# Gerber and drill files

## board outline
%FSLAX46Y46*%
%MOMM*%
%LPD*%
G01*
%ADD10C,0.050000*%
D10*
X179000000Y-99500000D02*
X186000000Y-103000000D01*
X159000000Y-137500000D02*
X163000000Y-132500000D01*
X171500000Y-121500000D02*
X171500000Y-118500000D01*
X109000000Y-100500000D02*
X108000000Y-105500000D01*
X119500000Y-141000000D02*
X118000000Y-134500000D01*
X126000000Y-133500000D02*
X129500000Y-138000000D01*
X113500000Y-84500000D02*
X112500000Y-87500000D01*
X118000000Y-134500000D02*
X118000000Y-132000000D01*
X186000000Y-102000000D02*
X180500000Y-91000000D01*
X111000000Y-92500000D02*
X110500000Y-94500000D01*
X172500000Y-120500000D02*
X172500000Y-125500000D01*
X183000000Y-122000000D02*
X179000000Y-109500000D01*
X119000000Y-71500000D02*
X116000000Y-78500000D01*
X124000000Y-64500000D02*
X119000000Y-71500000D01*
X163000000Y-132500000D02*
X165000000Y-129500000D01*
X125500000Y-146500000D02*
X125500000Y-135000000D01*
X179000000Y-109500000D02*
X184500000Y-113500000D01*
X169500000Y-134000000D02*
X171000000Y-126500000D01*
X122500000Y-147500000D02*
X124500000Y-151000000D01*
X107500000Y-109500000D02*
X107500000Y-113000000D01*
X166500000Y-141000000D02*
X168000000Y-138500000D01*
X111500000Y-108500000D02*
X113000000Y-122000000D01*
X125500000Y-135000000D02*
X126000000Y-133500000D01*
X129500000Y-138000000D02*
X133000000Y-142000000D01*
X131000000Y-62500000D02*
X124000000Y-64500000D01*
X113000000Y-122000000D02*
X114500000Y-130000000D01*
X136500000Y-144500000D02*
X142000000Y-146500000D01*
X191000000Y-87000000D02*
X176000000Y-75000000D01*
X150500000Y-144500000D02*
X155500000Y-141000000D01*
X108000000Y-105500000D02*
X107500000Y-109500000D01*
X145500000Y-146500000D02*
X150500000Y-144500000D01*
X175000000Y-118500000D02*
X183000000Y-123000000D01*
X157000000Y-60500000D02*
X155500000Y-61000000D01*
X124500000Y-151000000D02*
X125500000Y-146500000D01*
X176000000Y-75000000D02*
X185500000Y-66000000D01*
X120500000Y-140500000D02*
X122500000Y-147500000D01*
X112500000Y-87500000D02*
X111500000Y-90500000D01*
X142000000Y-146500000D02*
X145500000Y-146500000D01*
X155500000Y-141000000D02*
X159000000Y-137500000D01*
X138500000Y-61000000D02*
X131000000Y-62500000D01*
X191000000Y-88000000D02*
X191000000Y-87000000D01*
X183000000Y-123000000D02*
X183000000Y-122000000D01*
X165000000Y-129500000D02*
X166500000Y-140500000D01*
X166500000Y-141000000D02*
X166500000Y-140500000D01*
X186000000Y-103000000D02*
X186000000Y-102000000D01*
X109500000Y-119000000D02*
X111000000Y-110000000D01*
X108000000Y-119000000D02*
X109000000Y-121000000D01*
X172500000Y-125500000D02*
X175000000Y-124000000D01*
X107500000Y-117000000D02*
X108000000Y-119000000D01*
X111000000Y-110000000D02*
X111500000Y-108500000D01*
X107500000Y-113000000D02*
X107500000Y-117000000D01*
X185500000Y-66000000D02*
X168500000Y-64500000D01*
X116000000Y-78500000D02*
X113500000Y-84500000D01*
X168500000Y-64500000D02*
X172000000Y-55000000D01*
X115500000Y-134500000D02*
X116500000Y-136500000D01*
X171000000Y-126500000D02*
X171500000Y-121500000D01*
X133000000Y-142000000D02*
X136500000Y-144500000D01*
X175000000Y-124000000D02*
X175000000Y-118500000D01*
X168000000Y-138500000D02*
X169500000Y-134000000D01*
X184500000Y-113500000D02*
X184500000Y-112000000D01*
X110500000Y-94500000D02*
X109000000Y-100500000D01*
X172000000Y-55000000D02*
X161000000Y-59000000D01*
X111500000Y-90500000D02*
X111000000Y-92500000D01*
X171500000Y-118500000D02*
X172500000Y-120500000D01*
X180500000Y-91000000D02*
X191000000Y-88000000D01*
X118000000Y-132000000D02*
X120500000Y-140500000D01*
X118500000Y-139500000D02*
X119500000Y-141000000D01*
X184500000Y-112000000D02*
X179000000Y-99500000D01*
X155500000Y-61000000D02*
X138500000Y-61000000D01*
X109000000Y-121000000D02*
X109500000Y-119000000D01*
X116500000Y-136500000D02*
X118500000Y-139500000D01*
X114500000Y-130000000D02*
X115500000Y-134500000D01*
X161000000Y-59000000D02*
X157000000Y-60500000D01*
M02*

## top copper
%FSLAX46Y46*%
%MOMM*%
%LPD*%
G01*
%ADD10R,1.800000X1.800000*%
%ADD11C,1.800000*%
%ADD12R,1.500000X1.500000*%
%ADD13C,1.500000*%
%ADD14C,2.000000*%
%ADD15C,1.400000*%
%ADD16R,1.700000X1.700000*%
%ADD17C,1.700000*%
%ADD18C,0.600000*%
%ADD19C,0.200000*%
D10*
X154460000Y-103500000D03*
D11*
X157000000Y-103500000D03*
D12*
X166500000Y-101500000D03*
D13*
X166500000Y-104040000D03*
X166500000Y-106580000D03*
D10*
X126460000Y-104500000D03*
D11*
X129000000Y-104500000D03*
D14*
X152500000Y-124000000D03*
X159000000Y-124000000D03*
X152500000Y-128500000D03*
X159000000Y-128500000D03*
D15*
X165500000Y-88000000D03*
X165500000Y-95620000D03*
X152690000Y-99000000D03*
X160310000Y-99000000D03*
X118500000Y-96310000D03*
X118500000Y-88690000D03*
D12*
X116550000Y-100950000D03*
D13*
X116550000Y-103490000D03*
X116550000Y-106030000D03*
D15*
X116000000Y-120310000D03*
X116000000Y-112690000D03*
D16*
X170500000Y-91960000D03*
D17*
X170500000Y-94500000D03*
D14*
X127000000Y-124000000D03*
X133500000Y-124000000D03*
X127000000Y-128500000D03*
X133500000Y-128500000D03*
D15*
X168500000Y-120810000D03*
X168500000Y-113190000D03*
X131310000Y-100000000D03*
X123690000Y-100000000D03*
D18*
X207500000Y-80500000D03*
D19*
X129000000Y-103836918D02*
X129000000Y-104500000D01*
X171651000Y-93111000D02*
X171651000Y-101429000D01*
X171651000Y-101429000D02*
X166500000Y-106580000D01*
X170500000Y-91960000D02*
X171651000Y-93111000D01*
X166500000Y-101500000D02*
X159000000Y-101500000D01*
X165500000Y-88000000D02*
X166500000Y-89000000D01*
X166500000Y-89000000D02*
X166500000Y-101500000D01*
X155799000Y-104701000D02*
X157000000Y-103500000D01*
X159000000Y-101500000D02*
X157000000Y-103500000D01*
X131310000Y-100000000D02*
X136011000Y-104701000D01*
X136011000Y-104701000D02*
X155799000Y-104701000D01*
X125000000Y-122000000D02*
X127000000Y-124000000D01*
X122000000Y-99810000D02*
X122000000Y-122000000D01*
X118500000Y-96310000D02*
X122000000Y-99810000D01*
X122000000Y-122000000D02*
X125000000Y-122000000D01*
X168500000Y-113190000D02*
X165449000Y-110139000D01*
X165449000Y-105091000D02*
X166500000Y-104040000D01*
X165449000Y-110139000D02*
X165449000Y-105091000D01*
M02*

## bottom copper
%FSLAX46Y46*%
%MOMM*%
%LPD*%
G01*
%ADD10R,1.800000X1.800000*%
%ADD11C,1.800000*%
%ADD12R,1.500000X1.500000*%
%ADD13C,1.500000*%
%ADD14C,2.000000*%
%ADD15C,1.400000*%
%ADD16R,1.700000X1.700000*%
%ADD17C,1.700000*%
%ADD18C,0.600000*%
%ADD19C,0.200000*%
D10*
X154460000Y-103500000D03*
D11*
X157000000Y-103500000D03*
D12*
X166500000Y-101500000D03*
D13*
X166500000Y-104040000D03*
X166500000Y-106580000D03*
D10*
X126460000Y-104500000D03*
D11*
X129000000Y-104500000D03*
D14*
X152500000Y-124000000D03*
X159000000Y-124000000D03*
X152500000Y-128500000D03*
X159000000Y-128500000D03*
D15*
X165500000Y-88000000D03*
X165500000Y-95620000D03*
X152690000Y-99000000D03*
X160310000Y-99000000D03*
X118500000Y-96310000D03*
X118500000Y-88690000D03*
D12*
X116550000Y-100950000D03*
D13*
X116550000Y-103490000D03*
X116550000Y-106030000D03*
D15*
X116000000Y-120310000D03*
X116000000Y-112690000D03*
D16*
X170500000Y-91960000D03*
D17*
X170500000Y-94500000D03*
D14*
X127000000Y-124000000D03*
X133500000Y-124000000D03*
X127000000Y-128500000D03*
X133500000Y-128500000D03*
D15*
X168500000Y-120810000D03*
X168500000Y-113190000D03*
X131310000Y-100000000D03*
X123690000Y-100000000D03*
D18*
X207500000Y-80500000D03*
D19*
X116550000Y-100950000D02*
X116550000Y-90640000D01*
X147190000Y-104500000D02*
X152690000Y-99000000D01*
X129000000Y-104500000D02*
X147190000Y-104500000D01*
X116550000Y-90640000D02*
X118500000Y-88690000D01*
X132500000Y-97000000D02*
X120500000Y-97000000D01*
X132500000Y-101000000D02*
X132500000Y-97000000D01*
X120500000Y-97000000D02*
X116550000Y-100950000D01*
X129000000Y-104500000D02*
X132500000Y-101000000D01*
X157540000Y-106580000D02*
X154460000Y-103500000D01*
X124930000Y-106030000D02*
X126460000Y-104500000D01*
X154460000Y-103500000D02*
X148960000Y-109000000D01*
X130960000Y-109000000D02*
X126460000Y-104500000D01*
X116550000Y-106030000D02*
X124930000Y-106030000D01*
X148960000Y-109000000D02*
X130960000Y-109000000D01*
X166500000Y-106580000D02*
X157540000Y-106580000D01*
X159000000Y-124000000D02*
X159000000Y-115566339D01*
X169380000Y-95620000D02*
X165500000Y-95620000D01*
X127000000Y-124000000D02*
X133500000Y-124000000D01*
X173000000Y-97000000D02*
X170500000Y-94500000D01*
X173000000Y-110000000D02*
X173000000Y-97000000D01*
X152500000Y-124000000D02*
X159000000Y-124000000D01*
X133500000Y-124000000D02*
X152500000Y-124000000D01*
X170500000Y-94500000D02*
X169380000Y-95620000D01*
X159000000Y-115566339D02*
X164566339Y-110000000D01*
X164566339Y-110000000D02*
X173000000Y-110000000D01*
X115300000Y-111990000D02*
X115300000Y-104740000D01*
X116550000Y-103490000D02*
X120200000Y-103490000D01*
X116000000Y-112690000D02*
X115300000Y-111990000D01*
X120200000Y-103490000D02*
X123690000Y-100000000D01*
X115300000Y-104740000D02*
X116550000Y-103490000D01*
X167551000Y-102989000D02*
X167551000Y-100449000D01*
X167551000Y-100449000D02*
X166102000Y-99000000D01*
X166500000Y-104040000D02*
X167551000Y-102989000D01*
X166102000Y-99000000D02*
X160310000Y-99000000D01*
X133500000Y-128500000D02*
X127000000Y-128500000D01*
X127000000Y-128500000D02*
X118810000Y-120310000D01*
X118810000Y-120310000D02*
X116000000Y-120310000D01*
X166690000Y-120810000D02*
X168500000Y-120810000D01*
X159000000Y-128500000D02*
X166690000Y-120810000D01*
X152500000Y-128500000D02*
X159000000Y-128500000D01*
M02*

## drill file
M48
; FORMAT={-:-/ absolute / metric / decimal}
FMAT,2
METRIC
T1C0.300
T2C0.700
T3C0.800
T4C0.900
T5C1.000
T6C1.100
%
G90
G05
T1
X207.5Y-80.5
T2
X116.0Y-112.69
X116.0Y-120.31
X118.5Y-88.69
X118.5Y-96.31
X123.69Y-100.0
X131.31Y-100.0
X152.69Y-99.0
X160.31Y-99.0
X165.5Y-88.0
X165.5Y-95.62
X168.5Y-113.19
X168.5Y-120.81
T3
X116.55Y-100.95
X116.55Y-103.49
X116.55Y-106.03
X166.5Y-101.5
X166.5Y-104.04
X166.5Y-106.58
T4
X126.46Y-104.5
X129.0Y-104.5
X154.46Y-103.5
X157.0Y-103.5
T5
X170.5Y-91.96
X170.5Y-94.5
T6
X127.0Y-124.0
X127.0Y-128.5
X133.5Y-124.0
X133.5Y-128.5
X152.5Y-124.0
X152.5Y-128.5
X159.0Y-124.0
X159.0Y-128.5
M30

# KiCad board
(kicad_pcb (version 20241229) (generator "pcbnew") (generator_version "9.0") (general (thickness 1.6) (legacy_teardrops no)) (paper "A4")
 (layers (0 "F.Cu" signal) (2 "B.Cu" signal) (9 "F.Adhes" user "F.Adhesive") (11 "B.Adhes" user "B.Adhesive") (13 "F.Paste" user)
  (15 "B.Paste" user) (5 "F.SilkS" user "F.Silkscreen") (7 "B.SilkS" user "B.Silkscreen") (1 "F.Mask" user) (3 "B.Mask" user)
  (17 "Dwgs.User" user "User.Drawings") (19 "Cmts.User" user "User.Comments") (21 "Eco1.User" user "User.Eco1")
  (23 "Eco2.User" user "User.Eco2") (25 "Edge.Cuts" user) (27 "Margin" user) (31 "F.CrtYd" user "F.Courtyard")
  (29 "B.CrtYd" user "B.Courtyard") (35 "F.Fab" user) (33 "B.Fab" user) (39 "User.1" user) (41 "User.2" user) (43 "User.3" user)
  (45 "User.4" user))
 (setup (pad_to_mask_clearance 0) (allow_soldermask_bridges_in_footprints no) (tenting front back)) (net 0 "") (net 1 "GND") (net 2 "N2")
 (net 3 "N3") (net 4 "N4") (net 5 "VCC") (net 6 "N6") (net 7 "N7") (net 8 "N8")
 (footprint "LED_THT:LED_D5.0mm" (layer "F.Cu") (at 154.46 103.5)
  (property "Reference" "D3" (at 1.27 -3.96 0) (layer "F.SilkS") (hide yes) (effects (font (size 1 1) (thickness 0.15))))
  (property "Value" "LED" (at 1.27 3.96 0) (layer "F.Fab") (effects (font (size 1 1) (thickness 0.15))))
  (pad "1" thru_hole rect (at 0 0) (size 1.8 1.8) (drill 0.9) (layers "*.Cu" "*.Mask") (remove_unused_layers no) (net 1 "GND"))
  (pad "2" thru_hole circle (at 2.54 0) (size 1.8 1.8) (drill 0.9) (layers "*.Cu" "*.Mask") (remove_unused_layers no) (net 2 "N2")))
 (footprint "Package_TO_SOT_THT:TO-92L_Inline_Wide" (layer "F.Cu") (at 166.5 101.5 -90)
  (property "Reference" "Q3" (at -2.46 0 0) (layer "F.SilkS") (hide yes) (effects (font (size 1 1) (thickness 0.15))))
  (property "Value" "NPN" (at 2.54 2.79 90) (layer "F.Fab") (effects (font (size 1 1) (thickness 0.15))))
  (pad "1" thru_hole rect (at 0 0 270) (size 1.5 1.5) (drill 0.8) (layers "*.Cu" "*.Mask") (remove_unused_layers no) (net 2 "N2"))
  (pad "2" thru_hole circle (at 2.54 0 270) (size 1.5 1.5) (drill 0.8) (layers "*.Cu" "*.Mask") (remove_unused_layers no) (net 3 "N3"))
  (pad "3" thru_hole circle (at 5.08 0 270) (size 1.5 1.5) (drill 0.8) (layers "*.Cu" "*.Mask") (remove_unused_layers no) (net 1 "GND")))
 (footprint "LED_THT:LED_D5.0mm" (layer "F.Cu") (at 126.46 104.5)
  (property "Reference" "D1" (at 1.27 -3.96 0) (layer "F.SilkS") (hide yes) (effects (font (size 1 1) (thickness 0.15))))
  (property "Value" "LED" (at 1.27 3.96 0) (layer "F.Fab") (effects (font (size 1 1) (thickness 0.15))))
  (pad "1" thru_hole rect (at 0 0) (size 1.8 1.8) (drill 0.9) (layers "*.Cu" "*.Mask") (remove_unused_layers no) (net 1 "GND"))
  (pad "2" thru_hole circle (at 2.54 0) (size 1.8 1.8) (drill 0.9) (layers "*.Cu" "*.Mask") (remove_unused_layers no) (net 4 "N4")))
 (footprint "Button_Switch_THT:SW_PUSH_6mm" (layer "F.Cu") (at 152.5 124)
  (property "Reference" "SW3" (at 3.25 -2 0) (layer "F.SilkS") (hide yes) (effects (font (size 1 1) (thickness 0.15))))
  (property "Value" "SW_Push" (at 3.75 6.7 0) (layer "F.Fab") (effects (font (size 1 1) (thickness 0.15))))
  (pad "1" thru_hole circle (at 0 0 90) (size 2 2) (drill 1.1) (layers "*.Cu" "*.Mask") (remove_unused_layers no) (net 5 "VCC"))
  (pad "1" thru_hole circle (at 6.5 0 90) (size 2 2) (drill 1.1) (layers "*.Cu" "*.Mask") (remove_unused_layers no) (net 5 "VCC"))
  (pad "2" thru_hole circle (at 0 4.5 90) (size 2 2) (drill 1.1) (layers "*.Cu" "*.Mask") (remove_unused_layers no) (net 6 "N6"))
  (pad "2" thru_hole circle (at 6.5 4.5 90) (size 2 2) (drill 1.1) (layers "*.Cu" "*.Mask") (remove_unused_layers no) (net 6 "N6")))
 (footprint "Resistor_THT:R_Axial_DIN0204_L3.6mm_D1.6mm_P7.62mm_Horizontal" (layer "F.Cu") (at 165.5 88 -90)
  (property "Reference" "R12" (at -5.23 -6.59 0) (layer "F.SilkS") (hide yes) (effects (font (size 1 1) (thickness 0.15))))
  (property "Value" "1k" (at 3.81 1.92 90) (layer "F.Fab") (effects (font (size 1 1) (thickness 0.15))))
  (pad "1" thru_hole circle (at 0 0 270) (size 1.4 1.4) (drill 0.7) (layers "*.Cu" "*.Mask") (remove_unused_layers no) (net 2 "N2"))
  (pad "2" thru_hole circle (at 7.62 0 270) (size 1.4 1.4) (drill 0.7) (layers "*.Cu" "*.Mask") (remove_unused_layers no) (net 5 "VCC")))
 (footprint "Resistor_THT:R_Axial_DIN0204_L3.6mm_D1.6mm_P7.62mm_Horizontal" (layer "F.Cu") (at 152.69 99)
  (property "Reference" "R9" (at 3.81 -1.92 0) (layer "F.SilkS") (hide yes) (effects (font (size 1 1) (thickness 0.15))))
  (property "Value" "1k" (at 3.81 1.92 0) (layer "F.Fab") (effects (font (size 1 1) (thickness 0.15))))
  (pad "1" thru_hole circle (at 0 0) (size 1.4 1.4) (drill 0.7) (layers "*.Cu" "*.Mask") (remove_unused_layers no) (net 4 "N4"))
  (pad "2" thru_hole circle (at 7.62 0) (size 1.4 1.4) (drill 0.7) (layers "*.Cu" "*.Mask") (remove_unused_layers no) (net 3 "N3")))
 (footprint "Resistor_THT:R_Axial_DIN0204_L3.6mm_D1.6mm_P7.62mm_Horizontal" (layer "F.Cu") (at 118.5 96.31 90)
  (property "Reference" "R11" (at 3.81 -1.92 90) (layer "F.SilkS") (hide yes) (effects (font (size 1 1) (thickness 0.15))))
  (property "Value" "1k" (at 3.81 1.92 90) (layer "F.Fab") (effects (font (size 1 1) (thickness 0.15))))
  (pad "1" thru_hole circle (at 0 0 90) (size 1.4 1.4) (drill 0.7) (layers "*.Cu" "*.Mask") (remove_unused_layers no) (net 5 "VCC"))
  (pad "2" thru_hole circle (at 7.62 0 90) (size 1.4 1.4) (drill 0.7) (layers "*.Cu" "*.Mask") (remove_unused_layers no) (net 4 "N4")))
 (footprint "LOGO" (layer "F.Cu") (at 149.5 103)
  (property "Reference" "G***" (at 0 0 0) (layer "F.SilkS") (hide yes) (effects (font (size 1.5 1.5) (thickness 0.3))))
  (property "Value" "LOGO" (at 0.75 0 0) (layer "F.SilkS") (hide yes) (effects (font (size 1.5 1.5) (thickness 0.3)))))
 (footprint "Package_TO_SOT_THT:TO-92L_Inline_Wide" (layer "F.Cu") (at 116.55 100.95 -90)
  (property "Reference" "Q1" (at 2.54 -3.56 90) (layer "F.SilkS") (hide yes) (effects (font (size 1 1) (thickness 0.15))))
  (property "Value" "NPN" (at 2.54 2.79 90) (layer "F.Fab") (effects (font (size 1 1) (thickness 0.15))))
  (pad "1" thru_hole rect (at 0 0 270) (size 1.5 1.5) (drill 0.8) (layers "*.Cu" "*.Mask") (remove_unused_layers no) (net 4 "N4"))
  (pad "2" thru_hole circle (at 2.54 0 270) (size 1.5 1.5) (drill 0.8) (layers "*.Cu" "*.Mask") (remove_unused_layers no) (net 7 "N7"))
  (pad "3" thru_hole circle (at 5.08 0 270) (size 1.5 1.5) (drill 0.8) (layers "*.Cu" "*.Mask") (remove_unused_layers no) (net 1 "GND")))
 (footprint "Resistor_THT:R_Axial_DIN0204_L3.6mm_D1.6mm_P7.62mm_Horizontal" (layer "F.Cu") (at 116 120.31 90)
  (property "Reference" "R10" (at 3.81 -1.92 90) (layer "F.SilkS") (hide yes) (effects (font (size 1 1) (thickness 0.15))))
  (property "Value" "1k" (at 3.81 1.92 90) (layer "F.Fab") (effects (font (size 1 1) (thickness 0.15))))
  (pad "1" thru_hole circle (at 0 0 90) (size 1.4 1.4) (drill 0.7) (layers "*.Cu" "*.Mask") (remove_unused_layers no) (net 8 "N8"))
  (pad "2" thru_hole circle (at 7.62 0 90) (size 1.4 1.4) (drill 0.7) (layers "*.Cu" "*.Mask") (remove_unused_layers no) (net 7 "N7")))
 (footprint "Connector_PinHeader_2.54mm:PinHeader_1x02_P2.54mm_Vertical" (layer "F.Cu") (at 170.5 91.96)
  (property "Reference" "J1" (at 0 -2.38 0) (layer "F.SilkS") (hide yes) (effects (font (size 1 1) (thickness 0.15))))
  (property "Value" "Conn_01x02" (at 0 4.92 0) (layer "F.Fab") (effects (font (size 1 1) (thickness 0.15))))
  (pad "1" thru_hole rect (at 0 0) (size 1.7 1.7) (drill 1) (layers "*.Cu" "*.Mask") (remove_unused_layers no) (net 1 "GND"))
  (pad "2" thru_hole circle (at 0 2.54) (size 1.7 1.7) (drill 1) (layers "*.Cu" "*.Mask") (remove_unused_layers no) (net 5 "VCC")))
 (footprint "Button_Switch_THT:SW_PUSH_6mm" (layer "F.Cu") (at 127 124)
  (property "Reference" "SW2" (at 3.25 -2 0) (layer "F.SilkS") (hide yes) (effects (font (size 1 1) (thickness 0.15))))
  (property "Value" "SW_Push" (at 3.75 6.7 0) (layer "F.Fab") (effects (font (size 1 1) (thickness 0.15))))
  (pad "1" thru_hole circle (at 0 0 90) (size 2 2) (drill 1.1) (layers "*.Cu" "*.Mask") (remove_unused_layers no) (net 5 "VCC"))
  (pad "1" thru_hole circle (at 6.5 0 90) (size 2 2) (drill 1.1) (layers "*.Cu" "*.Mask") (remove_unused_layers no) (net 5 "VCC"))
  (pad "2" thru_hole circle (at 0 4.5 90) (size 2 2) (drill 1.1) (layers "*.Cu" "*.Mask") (remove_unused_layers no) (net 8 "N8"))
  (pad "2" thru_hole circle (at 6.5 4.5 90) (size 2 2) (drill 1.1) (layers "*.Cu" "*.Mask") (remove_unused_layers no) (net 8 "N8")))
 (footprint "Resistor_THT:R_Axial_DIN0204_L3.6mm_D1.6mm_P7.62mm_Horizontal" (layer "F.Cu") (at 168.5 120.81 90)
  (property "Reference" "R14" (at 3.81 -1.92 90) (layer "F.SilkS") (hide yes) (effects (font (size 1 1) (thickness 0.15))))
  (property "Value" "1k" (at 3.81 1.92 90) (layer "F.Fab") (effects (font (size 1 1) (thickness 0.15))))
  (pad "1" thru_hole circle (at 0 0 90) (size 1.4 1.4) (drill 0.7) (layers "*.Cu" "*.Mask") (remove_unused_layers no) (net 6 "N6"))
  (pad "2" thru_hole circle (at 7.62 0 90) (size 1.4 1.4) (drill 0.7) (layers "*.Cu" "*.Mask") (remove_unused_layers no) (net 3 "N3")))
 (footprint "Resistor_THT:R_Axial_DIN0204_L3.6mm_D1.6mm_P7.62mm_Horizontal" (layer "F.Cu") (at 131.31 100 180)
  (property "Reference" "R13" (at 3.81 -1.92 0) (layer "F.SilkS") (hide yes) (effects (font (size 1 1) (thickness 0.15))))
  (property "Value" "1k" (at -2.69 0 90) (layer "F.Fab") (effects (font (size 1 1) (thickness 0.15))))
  (pad "1" thru_hole circle (at 0 0 180) (size 1.4 1.4) (drill 0.7) (layers "*.Cu" "*.Mask") (remove_unused_layers no) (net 2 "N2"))
  (pad "2" thru_hole circle (at 7.62 0 180) (size 1.4 1.4) (drill 0.7) (layers "*.Cu" "*.Mask") (remove_unused_layers no) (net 7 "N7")))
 (gr_line (start 179 99.5) (end 186 103) (stroke (width 0.05) (type default)) (layer "Edge.Cuts"))
 (gr_line (start 159 137.5) (end 163 132.5) (stroke (width 0.05) (type default)) (layer "Edge.Cuts"))
 (gr_line (start 171.5 121.5) (end 171.5 118.5) (stroke (width 0.05) (type default)) (layer "Edge.Cuts"))
 (gr_line (start 109 100.5) (end 108 105.5) (stroke (width 0.05) (type default)) (layer "Edge.Cuts"))
 (gr_line (start 119.5 141) (end 118 134.5) (stroke (width 0.05) (type default)) (layer "Edge.Cuts"))
 (gr_line (start 126 133.5) (end 129.5 138) (stroke (width 0.05) (type default)) (layer "Edge.Cuts"))
 (gr_line (start 113.5 84.5) (end 112.5 87.5) (stroke (width 0.05) (type default)) (layer "Edge.Cuts"))
 (gr_line (start 118 134.5) (end 118 132) (stroke (width 0.05) (type default)) (layer "Edge.Cuts"))
 (gr_line (start 186 102) (end 180.5 91) (stroke (width 0.05) (type default)) (layer "Edge.Cuts"))
 (gr_line (start 111 92.5) (end 110.5 94.5) (stroke (width 0.05) (type default)) (layer "Edge.Cuts"))
 (gr_line (start 172.5 120.5) (end 172.5 125.5) (stroke (width 0.05) (type default)) (layer "Edge.Cuts"))
 (gr_line (start 183 122) (end 179 109.5) (stroke (width 0.05) (type default)) (layer "Edge.Cuts"))
 (gr_line (start 119 71.5) (end 116 78.5) (stroke (width 0.05) (type default)) (layer "Edge.Cuts"))
 (gr_line (start 124 64.5) (end 119 71.5) (stroke (width 0.05) (type default)) (layer "Edge.Cuts"))
 (gr_line (start 163 132.5) (end 165 129.5) (stroke (width 0.05) (type default)) (layer "Edge.Cuts"))
 (gr_line (start 125.5 146.5) (end 125.5 135) (stroke (width 0.05) (type default)) (layer "Edge.Cuts"))
 (gr_line (start 179 109.5) (end 184.5 113.5) (stroke (width 0.05) (type default)) (layer "Edge.Cuts"))
 (gr_line (start 169.5 134) (end 171 126.5) (stroke (width 0.05) (type default)) (layer "Edge.Cuts"))
 (gr_line (start 122.5 147.5) (end 124.5 151) (stroke (width 0.05) (type default)) (layer "Edge.Cuts"))
 (gr_line (start 107.5 109.5) (end 107.5 113) (stroke (width 0.05) (type default)) (layer "Edge.Cuts"))
 (gr_line (start 166.5 141) (end 168 138.5) (stroke (width 0.05) (type default)) (layer "Edge.Cuts"))
 (gr_line (start 111.5 108.5) (end 113 122) (stroke (width 0.05) (type default)) (layer "Edge.Cuts"))
 (gr_line (start 125.5 135) (end 126 133.5) (stroke (width 0.05) (type default)) (layer "Edge.Cuts"))
 (gr_line (start 129.5 138) (end 133 142) (stroke (width 0.05) (type default)) (layer "Edge.Cuts"))
 (gr_line (start 131 62.5) (end 124 64.5) (stroke (width 0.05) (type default)) (layer "Edge.Cuts"))
 (gr_line (start 113 122) (end 114.5 130) (stroke (width 0.05) (type default)) (layer "Edge.Cuts"))
 (gr_line (start 136.5 144.5) (end 142 146.5) (stroke (width 0.05) (type default)) (layer "Edge.Cuts"))
 (gr_line (start 191 87) (end 176 75) (stroke (width 0.05) (type default)) (layer "Edge.Cuts"))
 (gr_line (start 150.5 144.5) (end 155.5 141) (stroke (width 0.05) (type default)) (layer "Edge.Cuts"))
 (gr_line (start 108 105.5) (end 107.5 109.5) (stroke (width 0.05) (type default)) (layer "Edge.Cuts"))
 (gr_line (start 145.5 146.5) (end 150.5 144.5) (stroke (width 0.05) (type default)) (layer "Edge.Cuts"))
 (gr_line (start 175 118.5) (end 183 123) (stroke (width 0.05) (type default)) (layer "Edge.Cuts"))
 (gr_line (start 157 60.5) (end 155.5 61) (stroke (width 0.05) (type default)) (layer "Edge.Cuts"))
 (gr_line (start 124.5 151) (end 125.5 146.5) (stroke (width 0.05) (type default)) (layer "Edge.Cuts"))
 (gr_line (start 176 75) (end 185.5 66) (stroke (width 0.05) (type default)) (layer "Edge.Cuts"))
 (gr_line (start 120.5 140.5) (end 122.5 147.5) (stroke (width 0.05) (type default)) (layer "Edge.Cuts"))
 (gr_line (start 112.5 87.5) (end 111.5 90.5) (stroke (width 0.05) (type default)) (layer "Edge.Cuts"))
 (gr_line (start 142 146.5) (end 145.5 146.5) (stroke (width 0.05) (type default)) (layer "Edge.Cuts"))
 (gr_line (start 155.5 141) (end 159 137.5) (stroke (width 0.05) (type default)) (layer "Edge.Cuts"))
 (gr_line (start 138.5 61) (end 131 62.5) (stroke (width 0.05) (type default)) (layer "Edge.Cuts"))
 (gr_line (start 191 88) (end 191 87) (stroke (width 0.05) (type default)) (layer "Edge.Cuts"))
 (gr_line (start 183 123) (end 183 122) (stroke (width 0.05) (type default)) (layer "Edge.Cuts"))
 (gr_line (start 165 129.5) (end 166.5 140.5) (stroke (width 0.05) (type default)) (layer "Edge.Cuts"))
 (gr_line (start 166.5 141) (end 166.5 140.5) (stroke (width 0.05) (type default)) (layer "Edge.Cuts"))
 (gr_line (start 186 103) (end 186 102) (stroke (width 0.05) (type default)) (layer "Edge.Cuts"))
 (gr_line (start 109.5 119) (end 111 110) (stroke (width 0.05) (type default)) (layer "Edge.Cuts"))
 (gr_line (start 108 119) (end 109 121) (stroke (width 0.05) (type default)) (layer "Edge.Cuts"))
 (gr_line (start 172.5 125.5) (end 175 124) (stroke (width 0.05) (type default)) (layer "Edge.Cuts"))
 (gr_line (start 107.5 117) (end 108 119) (stroke (width 0.05) (type default)) (layer "Edge.Cuts"))
 (gr_line (start 111 110) (end 111.5 108.5) (stroke (width 0.05) (type default)) (layer "Edge.Cuts"))
 (gr_line (start 107.5 113) (end 107.5 117) (stroke (width 0.05) (type default)) (layer "Edge.Cuts"))
 (gr_line (start 185.5 66) (end 168.5 64.5) (stroke (width 0.05) (type default)) (layer "Edge.Cuts"))
 (gr_line (start 116 78.5) (end 113.5 84.5) (stroke (width 0.05) (type default)) (layer "Edge.Cuts"))
 (gr_line (start 168.5 64.5) (end 172 55) (stroke (width 0.05) (type default)) (layer "Edge.Cuts"))
 (gr_line (start 115.5 134.5) (end 116.5 136.5) (stroke (width 0.05) (type default)) (layer "Edge.Cuts"))
 (gr_line (start 171 126.5) (end 171.5 121.5) (stroke (width 0.05) (type default)) (layer "Edge.Cuts"))
 (gr_line (start 133 142) (end 136.5 144.5) (stroke (width 0.05) (type default)) (layer "Edge.Cuts"))
 (gr_line (start 175 124) (end 175 118.5) (stroke (width 0.05) (type default)) (layer "Edge.Cuts"))
 (gr_line (start 168 138.5) (end 169.5 134) (stroke (width 0.05) (type default)) (layer "Edge.Cuts"))
 (gr_line (start 184.5 113.5) (end 184.5 112) (stroke (width 0.05) (type default)) (layer "Edge.Cuts"))
 (gr_line (start 110.5 94.5) (end 109 100.5) (stroke (width 0.05) (type default)) (layer "Edge.Cuts"))
 (gr_line (start 172 55) (end 161 59) (stroke (width 0.05) (type default)) (layer "Edge.Cuts"))
 (gr_line (start 111.5 90.5) (end 111 92.5) (stroke (width 0.05) (type default)) (layer "Edge.Cuts"))
 (gr_line (start 171.5 118.5) (end 172.5 120.5) (stroke (width 0.05) (type default)) (layer "Edge.Cuts"))
 (gr_line (start 180.5 91) (end 191 88) (stroke (width 0.05) (type default)) (layer "Edge.Cuts"))
 (gr_line (start 118 132) (end 120.5 140.5) (stroke (width 0.05) (type default)) (layer "Edge.Cuts"))
 (gr_line (start 118.5 139.5) (end 119.5 141) (stroke (width 0.05) (type default)) (layer "Edge.Cuts"))
 (gr_line (start 184.5 112) (end 179 99.5) (stroke (width 0.05) (type default)) (layer "Edge.Cuts"))
 (gr_line (start 155.5 61) (end 138.5 61) (stroke (width 0.05) (type default)) (layer "Edge.Cuts"))
 (gr_line (start 109 121) (end 109.5 119) (stroke (width 0.05) (type default)) (layer "Edge.Cuts"))
 (gr_line (start 116.5 136.5) (end 118.5 139.5) (stroke (width 0.05) (type default)) (layer "Edge.Cuts"))
 (gr_line (start 114.5 130) (end 115.5 134.5) (stroke (width 0.05) (type default)) (layer "Edge.Cuts"))
 (gr_line (start 161 59) (end 157 60.5) (stroke (width 0.05) (type default)) (layer "Edge.Cuts"))
 (via (at 207.5 80.5) (size 0.6) (drill 0.3) (layers "F.Cu" "B.Cu") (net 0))
 (segment (start 129 103.836918) (end 129 104.5) (width 0.2) (layer "F.Cu") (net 4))
 (segment (start 116.55 100.95) (end 116.55 90.64) (width 0.2) (layer "B.Cu") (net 4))
 (segment (start 147.19 104.5) (end 152.69 99) (width 0.2) (layer "B.Cu") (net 4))
 (segment (start 129 104.5) (end 147.19 104.5) (width 0.2) (layer "B.Cu") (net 4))
 (segment (start 116.55 90.64) (end 118.5 88.69) (width 0.2) (layer "B.Cu") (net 4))
 (segment (start 132.5 97) (end 120.5 97) (width 0.2) (layer "B.Cu") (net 4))
 (segment (start 132.5 101) (end 132.5 97) (width 0.2) (layer "B.Cu") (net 4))
 (segment (start 120.5 97) (end 116.55 100.95) (width 0.2) (layer "B.Cu") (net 4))
 (segment (start 129 104.5) (end 132.5 101) (width 0.2) (layer "B.Cu") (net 4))
 (segment (start 171.651 93.111) (end 171.651 101.429) (width 0.2) (layer "F.Cu") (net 1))
 (segment (start 171.651 101.429) (end 166.5 106.58) (width 0.2) (layer "F.Cu") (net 1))
 (segment (start 170.5 91.96) (end 171.651 93.111) (width 0.2) (layer "F.Cu") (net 1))
 (segment (start 157.54 106.58) (end 154.46 103.5) (width 0.2) (layer "B.Cu") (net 1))
 (segment (start 124.93 106.03) (end 126.46 104.5) (width 0.2) (layer "B.Cu") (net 1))
 (segment (start 154.46 103.5) (end 148.96 109) (width 0.2) (layer "B.Cu") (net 1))
 (segment (start 130.96 109) (end 126.46 104.5) (width 0.2) (layer "B.Cu") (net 1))
 (segment (start 116.55 106.03) (end 124.93 106.03) (width 0.2) (layer "B.Cu") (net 1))
 (segment (start 148.96 109) (end 130.96 109) (width 0.2) (layer "B.Cu") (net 1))
 (segment (start 166.5 106.58) (end 157.54 106.58) (width 0.2) (layer "B.Cu") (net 1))
 (segment (start 166.5 101.5) (end 159 101.5) (width 0.2) (layer "F.Cu") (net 2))
 (segment (start 165.5 88) (end 166.5 89) (width 0.2) (layer "F.Cu") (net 2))
 (segment (start 166.5 89) (end 166.5 101.5) (width 0.2) (layer "F.Cu") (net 2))
 (segment (start 155.799 104.701) (end 157 103.5) (width 0.2) (layer "F.Cu") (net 2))
 (segment (start 159 101.5) (end 157 103.5) (width 0.2) (layer "F.Cu") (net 2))
 (segment (start 131.31 100) (end 136.011 104.701) (width 0.2) (layer "F.Cu") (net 2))
 (segment (start 136.011 104.701) (end 155.799 104.701) (width 0.2) (layer "F.Cu") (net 2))
 (segment (start 125 122) (end 127 124) (width 0.2) (layer "F.Cu") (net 5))
 (segment (start 122 99.81) (end 122 122) (width 0.2) (layer "F.Cu") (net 5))
 (segment (start 118.5 96.31) (end 122 99.81) (width 0.2) (layer "F.Cu") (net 5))
 (segment (start 122 122) (end 125 122) (width 0.2) (layer "F.Cu") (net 5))
 (segment (start 159 124) (end 159 115.566339) (width 0.2) (layer "B.Cu") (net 5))
 (segment (start 169.38 95.62) (end 165.5 95.62) (width 0.2) (layer "B.Cu") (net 5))
 (segment (start 127 124) (end 133.5 124) (width 0.2) (layer "B.Cu") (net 5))
 (segment (start 173 97) (end 170.5 94.5) (width 0.2) (layer "B.Cu") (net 5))
 (segment (start 173 110) (end 173 97) (width 0.2) (layer "B.Cu") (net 5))
 (segment (start 152.5 124) (end 159 124) (width 0.2) (layer "B.Cu") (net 5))
 (segment (start 133.5 124) (end 152.5 124) (width 0.2) (layer "B.Cu") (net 5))
 (segment (start 170.5 94.5) (end 169.38 95.62) (width 0.2) (layer "B.Cu") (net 5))
 (segment (start 159 115.566339) (end 164.566339 110) (width 0.2) (layer "B.Cu") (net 5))
 (segment (start 164.566339 110) (end 173 110) (width 0.2) (layer "B.Cu") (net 5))
 (segment (start 115.3 111.99) (end 115.3 104.74) (width 0.2) (layer "B.Cu") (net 7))
 (segment (start 116.55 103.49) (end 120.2 103.49) (width 0.2) (layer "B.Cu") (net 7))
 (segment (start 116 112.69) (end 115.3 111.99) (width 0.2) (layer "B.Cu") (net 7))
 (segment (start 120.2 103.49) (end 123.69 100) (width 0.2) (layer "B.Cu") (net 7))
 (segment (start 115.3 104.74) (end 116.55 103.49) (width 0.2) (layer "B.Cu") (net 7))
 (segment (start 168.5 113.19) (end 165.449 110.139) (width 0.2) (layer "F.Cu") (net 3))
 (segment (start 165.449 105.091) (end 166.5 104.04) (width 0.2) (layer "F.Cu") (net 3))
 (segment (start 165.449 110.139) (end 165.449 105.091) (width 0.2) (layer "F.Cu") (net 3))
 (segment (start 167.551 102.989) (end 167.551 100.449) (width 0.2) (layer "B.Cu") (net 3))
 (segment (start 167.551 100.449) (end 166.102 99) (width 0.2) (layer "B.Cu") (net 3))
 (segment (start 166.5 104.04) (end 167.551 102.989) (width 0.2) (layer "B.Cu") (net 3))
 (segment (start 166.102 99) (end 160.31 99) (width 0.2) (layer "B.Cu") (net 3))
 (segment (start 133.5 128.5) (end 127 128.5) (width 0.2) (layer "B.Cu") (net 8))
 (segment (start 127 128.5) (end 118.81 120.31) (width 0.2) (layer "B.Cu") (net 8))
 (segment (start 118.81 120.31) (end 116 120.31) (width 0.2) (layer "B.Cu") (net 8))
 (segment (start 166.69 120.81) (end 168.5 120.81) (width 0.2) (layer "B.Cu") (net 6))
 (segment (start 159 128.5) (end 166.69 120.81) (width 0.2) (layer "B.Cu") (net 6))
 (segment (start 152.5 128.5) (end 159 128.5) (width 0.2) (layer "B.Cu") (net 6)))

